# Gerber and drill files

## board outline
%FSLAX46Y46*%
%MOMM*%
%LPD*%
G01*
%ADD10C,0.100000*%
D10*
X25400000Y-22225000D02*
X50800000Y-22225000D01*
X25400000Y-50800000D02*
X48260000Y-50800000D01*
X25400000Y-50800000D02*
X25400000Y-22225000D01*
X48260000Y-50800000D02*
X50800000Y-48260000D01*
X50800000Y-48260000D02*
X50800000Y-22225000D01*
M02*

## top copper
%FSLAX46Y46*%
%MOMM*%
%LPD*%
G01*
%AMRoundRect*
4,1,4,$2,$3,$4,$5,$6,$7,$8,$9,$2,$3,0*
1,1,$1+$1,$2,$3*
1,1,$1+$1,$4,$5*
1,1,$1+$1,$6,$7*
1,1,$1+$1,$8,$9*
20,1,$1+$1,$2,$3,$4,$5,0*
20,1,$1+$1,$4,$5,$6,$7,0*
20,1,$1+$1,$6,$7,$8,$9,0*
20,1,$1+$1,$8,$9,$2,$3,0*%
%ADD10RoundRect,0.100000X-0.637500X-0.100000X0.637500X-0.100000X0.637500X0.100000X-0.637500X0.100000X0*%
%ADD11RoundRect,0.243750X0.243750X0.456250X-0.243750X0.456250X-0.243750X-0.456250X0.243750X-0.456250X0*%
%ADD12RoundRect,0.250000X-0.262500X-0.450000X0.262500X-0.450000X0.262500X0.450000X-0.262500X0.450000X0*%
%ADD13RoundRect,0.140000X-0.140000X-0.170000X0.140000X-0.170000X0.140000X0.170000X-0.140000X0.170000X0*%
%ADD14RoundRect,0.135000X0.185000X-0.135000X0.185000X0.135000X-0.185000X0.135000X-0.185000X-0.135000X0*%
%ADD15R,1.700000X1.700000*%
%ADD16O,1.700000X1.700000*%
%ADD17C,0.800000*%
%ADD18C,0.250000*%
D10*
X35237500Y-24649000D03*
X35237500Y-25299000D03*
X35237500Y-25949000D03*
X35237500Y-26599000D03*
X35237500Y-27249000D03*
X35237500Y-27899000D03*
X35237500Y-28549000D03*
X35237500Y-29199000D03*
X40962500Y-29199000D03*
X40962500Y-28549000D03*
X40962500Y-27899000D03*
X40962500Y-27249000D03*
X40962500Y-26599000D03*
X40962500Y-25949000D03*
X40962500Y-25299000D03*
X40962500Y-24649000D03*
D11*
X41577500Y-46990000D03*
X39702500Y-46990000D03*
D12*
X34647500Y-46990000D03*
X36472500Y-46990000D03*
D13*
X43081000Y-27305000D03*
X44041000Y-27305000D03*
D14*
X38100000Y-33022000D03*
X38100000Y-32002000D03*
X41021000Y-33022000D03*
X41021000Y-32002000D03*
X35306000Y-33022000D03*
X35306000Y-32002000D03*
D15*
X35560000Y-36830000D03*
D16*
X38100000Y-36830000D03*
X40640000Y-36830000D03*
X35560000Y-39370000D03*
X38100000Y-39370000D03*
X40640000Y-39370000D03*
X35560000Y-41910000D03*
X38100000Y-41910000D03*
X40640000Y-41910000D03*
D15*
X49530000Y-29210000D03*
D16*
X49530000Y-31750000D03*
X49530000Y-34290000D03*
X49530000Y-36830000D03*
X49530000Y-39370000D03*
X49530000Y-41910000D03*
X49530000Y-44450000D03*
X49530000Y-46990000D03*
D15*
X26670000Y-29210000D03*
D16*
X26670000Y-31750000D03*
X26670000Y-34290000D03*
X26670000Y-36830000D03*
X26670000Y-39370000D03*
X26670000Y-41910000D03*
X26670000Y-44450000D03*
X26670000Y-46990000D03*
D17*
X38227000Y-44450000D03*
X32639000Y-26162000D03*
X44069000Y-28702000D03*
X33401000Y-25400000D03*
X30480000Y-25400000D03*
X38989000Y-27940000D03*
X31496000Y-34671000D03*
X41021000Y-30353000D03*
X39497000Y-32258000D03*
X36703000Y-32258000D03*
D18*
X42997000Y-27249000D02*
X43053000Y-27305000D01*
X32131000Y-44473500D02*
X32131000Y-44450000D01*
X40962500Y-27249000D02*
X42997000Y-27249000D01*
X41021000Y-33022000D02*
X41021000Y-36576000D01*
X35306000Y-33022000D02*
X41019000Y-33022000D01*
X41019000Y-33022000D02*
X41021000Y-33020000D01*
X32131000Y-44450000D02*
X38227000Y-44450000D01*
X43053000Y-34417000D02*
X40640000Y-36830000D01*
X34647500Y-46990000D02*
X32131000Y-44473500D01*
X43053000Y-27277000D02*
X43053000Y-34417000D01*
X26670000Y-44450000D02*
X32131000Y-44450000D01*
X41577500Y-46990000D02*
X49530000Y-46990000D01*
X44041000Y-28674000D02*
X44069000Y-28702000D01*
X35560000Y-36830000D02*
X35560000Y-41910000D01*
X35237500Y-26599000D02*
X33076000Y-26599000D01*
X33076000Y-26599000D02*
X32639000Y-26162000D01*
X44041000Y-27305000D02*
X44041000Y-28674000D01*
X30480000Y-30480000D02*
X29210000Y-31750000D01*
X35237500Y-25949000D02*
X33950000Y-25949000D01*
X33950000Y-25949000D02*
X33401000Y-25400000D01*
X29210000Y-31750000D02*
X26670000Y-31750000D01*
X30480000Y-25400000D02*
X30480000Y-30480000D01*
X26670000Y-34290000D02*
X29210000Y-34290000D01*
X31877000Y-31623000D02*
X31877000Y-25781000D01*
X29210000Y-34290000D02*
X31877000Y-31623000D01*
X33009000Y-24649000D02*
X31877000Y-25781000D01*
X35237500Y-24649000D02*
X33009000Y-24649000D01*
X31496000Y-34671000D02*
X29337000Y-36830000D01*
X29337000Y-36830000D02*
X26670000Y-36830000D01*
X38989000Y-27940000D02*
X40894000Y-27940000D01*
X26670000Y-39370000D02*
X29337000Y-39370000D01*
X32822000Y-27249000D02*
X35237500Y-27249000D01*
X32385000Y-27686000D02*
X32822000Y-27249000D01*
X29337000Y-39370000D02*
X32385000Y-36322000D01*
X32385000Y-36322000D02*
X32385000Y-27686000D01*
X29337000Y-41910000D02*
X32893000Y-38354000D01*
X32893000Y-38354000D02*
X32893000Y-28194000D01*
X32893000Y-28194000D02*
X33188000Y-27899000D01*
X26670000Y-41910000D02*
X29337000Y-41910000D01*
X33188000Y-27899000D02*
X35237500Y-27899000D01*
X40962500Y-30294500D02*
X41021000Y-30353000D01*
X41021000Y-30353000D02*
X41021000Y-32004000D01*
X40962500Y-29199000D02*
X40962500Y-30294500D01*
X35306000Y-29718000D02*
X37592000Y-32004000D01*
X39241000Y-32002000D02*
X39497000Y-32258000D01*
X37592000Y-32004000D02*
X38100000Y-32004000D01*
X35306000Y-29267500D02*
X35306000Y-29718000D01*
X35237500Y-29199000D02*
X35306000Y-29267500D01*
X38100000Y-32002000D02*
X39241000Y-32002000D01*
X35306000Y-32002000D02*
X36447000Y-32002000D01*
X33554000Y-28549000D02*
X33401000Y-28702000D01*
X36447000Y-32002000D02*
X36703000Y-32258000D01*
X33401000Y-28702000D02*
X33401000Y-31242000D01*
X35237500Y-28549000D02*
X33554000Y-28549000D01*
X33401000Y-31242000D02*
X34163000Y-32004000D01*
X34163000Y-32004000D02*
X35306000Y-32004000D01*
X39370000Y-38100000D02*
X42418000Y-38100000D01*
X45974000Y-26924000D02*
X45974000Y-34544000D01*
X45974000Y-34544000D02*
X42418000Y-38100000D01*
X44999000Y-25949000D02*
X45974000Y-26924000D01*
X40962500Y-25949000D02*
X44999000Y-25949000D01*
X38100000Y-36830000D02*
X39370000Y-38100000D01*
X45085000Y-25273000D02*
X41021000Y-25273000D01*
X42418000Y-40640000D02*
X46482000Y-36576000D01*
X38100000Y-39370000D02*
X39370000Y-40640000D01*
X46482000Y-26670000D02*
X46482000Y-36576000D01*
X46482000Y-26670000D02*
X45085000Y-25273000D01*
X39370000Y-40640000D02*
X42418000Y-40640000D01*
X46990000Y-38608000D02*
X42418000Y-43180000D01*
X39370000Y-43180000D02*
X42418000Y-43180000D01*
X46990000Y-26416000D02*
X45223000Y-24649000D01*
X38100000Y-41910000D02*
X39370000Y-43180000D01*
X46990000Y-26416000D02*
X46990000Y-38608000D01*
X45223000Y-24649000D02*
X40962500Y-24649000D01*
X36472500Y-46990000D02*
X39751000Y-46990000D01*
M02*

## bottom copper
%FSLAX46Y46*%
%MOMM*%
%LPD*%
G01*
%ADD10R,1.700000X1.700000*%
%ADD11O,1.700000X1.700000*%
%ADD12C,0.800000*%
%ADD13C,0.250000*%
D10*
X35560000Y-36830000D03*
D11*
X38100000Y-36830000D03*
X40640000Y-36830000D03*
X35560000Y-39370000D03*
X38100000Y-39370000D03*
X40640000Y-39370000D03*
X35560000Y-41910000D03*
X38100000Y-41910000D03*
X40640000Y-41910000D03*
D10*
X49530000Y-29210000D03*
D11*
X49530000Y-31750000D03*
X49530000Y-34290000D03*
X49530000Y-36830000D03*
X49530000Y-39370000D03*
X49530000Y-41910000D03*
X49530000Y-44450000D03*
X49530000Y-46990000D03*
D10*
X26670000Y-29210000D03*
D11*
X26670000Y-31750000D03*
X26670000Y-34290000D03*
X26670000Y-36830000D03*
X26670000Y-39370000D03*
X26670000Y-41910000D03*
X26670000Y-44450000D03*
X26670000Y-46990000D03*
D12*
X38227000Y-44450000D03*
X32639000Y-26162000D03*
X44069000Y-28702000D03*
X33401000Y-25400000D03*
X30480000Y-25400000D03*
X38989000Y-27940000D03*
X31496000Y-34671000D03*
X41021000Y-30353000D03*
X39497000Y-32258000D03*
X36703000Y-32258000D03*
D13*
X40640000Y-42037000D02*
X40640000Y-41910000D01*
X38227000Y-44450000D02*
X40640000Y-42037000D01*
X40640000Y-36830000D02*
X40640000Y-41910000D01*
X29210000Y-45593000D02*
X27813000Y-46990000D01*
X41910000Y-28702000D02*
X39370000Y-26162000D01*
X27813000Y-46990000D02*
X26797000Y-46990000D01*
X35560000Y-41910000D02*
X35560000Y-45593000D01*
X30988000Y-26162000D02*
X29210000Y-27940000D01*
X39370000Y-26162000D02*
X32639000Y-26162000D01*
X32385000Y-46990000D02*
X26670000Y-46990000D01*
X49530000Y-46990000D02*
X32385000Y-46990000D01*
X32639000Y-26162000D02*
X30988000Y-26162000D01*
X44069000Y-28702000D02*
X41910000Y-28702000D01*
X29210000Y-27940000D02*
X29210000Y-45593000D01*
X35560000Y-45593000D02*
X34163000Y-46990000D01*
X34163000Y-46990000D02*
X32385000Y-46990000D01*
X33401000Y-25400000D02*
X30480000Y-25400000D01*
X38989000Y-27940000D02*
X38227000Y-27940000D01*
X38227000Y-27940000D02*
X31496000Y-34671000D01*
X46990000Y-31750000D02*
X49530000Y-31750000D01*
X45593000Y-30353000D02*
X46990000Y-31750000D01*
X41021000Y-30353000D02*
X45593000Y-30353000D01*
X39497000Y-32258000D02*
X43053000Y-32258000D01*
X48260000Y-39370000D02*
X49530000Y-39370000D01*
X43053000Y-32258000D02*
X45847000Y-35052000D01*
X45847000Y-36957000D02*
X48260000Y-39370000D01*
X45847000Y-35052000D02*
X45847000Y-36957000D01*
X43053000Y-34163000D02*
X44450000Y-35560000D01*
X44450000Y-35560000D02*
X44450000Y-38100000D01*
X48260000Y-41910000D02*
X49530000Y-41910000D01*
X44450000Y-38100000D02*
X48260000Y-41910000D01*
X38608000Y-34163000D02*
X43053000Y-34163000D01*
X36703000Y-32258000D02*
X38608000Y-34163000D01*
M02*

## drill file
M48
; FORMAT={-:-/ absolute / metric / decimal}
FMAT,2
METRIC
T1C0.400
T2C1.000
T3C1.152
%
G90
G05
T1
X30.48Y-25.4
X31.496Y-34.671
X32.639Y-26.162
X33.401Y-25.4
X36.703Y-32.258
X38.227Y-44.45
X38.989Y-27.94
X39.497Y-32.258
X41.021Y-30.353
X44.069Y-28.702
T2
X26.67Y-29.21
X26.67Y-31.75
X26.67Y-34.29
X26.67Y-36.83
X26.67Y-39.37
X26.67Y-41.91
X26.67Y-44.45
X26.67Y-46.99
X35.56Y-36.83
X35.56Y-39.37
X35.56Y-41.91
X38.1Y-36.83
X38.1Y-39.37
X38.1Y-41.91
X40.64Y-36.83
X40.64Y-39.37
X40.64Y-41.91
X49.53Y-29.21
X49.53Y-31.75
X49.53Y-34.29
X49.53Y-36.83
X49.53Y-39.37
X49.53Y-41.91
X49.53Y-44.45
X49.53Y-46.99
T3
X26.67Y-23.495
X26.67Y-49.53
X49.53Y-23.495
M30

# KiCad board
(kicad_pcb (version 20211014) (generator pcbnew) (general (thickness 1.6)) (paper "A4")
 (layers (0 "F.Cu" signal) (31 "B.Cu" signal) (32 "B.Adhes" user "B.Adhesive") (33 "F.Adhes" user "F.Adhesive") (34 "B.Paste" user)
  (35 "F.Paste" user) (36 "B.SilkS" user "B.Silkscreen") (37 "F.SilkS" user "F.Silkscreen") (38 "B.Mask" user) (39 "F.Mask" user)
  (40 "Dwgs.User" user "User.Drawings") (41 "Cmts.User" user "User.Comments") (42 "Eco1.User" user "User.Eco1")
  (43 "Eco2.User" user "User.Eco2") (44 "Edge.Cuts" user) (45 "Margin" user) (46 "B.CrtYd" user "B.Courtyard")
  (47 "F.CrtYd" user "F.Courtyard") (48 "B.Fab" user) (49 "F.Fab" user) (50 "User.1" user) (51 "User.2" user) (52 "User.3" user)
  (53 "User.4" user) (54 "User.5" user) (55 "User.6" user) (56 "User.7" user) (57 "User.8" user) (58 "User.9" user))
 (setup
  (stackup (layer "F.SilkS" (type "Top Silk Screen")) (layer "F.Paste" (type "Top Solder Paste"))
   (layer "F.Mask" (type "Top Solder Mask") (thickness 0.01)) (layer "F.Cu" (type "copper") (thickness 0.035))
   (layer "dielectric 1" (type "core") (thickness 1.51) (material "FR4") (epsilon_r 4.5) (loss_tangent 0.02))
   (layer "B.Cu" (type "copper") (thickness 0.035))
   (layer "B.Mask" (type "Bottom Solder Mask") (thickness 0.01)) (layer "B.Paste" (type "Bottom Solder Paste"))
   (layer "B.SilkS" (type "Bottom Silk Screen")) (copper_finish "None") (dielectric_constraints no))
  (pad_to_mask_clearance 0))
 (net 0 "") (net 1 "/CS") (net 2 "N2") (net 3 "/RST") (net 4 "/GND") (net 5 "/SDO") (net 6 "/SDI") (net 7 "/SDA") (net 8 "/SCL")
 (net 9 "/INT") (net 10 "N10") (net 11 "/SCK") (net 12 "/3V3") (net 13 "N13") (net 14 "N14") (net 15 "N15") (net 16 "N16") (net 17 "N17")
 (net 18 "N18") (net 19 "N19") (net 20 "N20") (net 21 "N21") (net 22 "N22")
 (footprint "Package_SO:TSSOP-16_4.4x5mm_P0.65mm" (layer "F.Cu") (at 38.1 26.924)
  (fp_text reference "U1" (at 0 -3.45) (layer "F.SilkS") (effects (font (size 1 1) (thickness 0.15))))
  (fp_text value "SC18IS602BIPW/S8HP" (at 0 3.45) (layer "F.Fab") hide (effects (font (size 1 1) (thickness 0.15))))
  (pad "1" smd roundrect (at -2.8625 -2.275) (size 1.475 0.4) (layers "F.Cu" "F.Paste" "F.Mask") (roundrect_rratio 0.25) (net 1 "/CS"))
  (pad "2" smd roundrect (at -2.8625 -1.625) (size 1.475 0.4) (layers "F.Cu" "F.Paste" "F.Mask") (roundrect_rratio 0.25) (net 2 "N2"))
  (pad "3" smd roundrect (at -2.8625 -0.975) (size 1.475 0.4) (layers "F.Cu" "F.Paste" "F.Mask") (roundrect_rratio 0.25) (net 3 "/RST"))
  (pad "4" smd roundrect (at -2.8625 -0.325) (size 1.475 0.4) (layers "F.Cu" "F.Paste" "F.Mask") (roundrect_rratio 0.25) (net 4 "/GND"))
  (pad "5" smd roundrect (at -2.8625 0.325) (size 1.475 0.4) (layers "F.Cu" "F.Paste" "F.Mask") (roundrect_rratio 0.25) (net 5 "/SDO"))
  (pad "6" smd roundrect (at -2.8625 0.975) (size 1.475 0.4) (layers "F.Cu" "F.Paste" "F.Mask") (roundrect_rratio 0.25) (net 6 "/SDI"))
  (pad "7" smd roundrect (at -2.8625 1.625) (size 1.475 0.4) (layers "F.Cu" "F.Paste" "F.Mask") (roundrect_rratio 0.25) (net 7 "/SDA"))
  (pad "8" smd roundrect (at -2.8625 2.275) (size 1.475 0.4) (layers "F.Cu" "F.Paste" "F.Mask") (roundrect_rratio 0.25) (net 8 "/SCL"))
  (pad "9" smd roundrect (at 2.8625 2.275) (size 1.475 0.4) (layers "F.Cu" "F.Paste" "F.Mask") (roundrect_rratio 0.25) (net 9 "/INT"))
  (pad "10" smd roundrect (at 2.8625 1.625) (size 1.475 0.4) (layers "F.Cu" "F.Paste" "F.Mask") (roundrect_rratio 0.25) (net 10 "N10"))
  (pad "11" smd roundrect (at 2.8625 0.975) (size 1.475 0.4) (layers "F.Cu" "F.Paste" "F.Mask") (roundrect_rratio 0.25) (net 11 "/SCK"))
  (pad "12" smd roundrect (at 2.8625 0.325) (size 1.475 0.4) (layers "F.Cu" "F.Paste" "F.Mask") (roundrect_rratio 0.25) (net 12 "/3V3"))
  (pad "13" smd roundrect (at 2.8625 -0.325) (size 1.475 0.4) (layers "F.Cu" "F.Paste" "F.Mask") (roundrect_rratio 0.25) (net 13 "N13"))
  (pad "14" smd roundrect (at 2.8625 -0.975) (size 1.475 0.4) (layers "F.Cu" "F.Paste" "F.Mask") (roundrect_rratio 0.25) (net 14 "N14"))
  (pad "15" smd roundrect (at 2.8625 -1.625) (size 1.475 0.4) (layers "F.Cu" "F.Paste" "F.Mask") (roundrect_rratio 0.25) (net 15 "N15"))
  (pad "16" smd roundrect (at 2.8625 -2.275) (size 1.475 0.4) (layers "F.Cu" "F.Paste" "F.Mask") (roundrect_rratio 0.25) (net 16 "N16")))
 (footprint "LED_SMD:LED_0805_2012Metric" (layer "F.Cu") (at 40.64 46.99 180)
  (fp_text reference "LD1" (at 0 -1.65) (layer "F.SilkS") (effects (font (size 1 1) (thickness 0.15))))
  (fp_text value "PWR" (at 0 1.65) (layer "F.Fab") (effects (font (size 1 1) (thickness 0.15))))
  (pad "1" smd roundrect (at -0.9375 0 180) (size 0.975 1.4) (layers "F.Cu" "F.Paste" "F.Mask") (roundrect_rratio 0.25) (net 4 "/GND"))
  (pad "2" smd roundrect (at 0.9375 0 180) (size 0.975 1.4) (layers "F.Cu" "F.Paste" "F.Mask") (roundrect_rratio 0.25) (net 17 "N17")))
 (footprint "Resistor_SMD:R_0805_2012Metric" (layer "F.Cu") (at 35.56 46.99)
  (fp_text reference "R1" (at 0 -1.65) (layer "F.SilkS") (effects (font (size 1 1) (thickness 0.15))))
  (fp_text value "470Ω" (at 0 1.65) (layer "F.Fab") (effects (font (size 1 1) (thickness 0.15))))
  (pad "1" smd roundrect (at -0.9125 0) (size 1.025 1.4) (layers "F.Cu" "F.Paste" "F.Mask") (roundrect_rratio 0.243902) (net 12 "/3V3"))
  (pad "2" smd roundrect (at 0.9125 0) (size 1.025 1.4) (layers "F.Cu" "F.Paste" "F.Mask") (roundrect_rratio 0.243902) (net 17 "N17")))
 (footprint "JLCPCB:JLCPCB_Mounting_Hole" (layer "F.Cu") (at 49.53 23.495)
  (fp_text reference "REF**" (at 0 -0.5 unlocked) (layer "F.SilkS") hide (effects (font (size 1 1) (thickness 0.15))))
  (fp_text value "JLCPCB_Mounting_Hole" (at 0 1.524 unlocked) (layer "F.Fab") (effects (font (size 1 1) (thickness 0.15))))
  (pad "" np_thru_hole circle (at 0 0) (size 1.152 1.152) (drill 1.152) (layers F&B.Cu *.Mask) (solder_mask_margin 0.148)))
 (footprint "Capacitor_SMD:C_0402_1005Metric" (layer "F.Cu") (at 43.561 27.305)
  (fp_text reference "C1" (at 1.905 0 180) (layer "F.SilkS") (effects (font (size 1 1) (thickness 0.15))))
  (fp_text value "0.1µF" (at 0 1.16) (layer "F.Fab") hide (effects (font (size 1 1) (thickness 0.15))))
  (pad "1" smd roundrect (at -0.48 0) (size 0.56 0.62) (layers "F.Cu" "F.Paste" "F.Mask") (roundrect_rratio 0.25) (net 12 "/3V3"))
  (pad "2" smd roundrect (at 0.48 0) (size 0.56 0.62) (layers "F.Cu" "F.Paste" "F.Mask") (roundrect_rratio 0.25) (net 4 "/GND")))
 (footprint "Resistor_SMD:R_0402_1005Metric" (layer "F.Cu") (at 38.1 32.512 90)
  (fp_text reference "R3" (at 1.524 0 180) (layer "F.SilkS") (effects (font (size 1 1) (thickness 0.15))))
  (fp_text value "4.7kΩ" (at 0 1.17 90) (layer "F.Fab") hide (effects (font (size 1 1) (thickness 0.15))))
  (pad "1" smd roundrect (at -0.51 0 90) (size 0.54 0.64) (layers "F.Cu" "F.Paste" "F.Mask") (roundrect_rratio 0.25) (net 12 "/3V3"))
  (pad "2" smd roundrect (at 0.51 0 90) (size 0.54 0.64) (layers "F.Cu" "F.Paste" "F.Mask") (roundrect_rratio 0.25) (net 8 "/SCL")))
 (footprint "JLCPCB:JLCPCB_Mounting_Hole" (layer "F.Cu") (at 26.67 23.495)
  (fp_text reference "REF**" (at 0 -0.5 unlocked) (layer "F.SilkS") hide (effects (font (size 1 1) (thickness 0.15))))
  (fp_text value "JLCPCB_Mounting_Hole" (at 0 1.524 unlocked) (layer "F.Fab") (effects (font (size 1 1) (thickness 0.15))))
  (pad "" np_thru_hole circle (at 0 0) (size 1.152 1.152) (drill 1.152) (layers F&B.Cu *.Mask) (solder_mask_margin 0.148)))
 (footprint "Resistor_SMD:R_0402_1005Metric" (layer "F.Cu") (at 41.021 32.512 90)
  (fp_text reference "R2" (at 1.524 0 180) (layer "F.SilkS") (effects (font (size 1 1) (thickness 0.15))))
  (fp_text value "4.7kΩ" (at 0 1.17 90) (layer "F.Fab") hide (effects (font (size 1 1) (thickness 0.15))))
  (pad "1" smd roundrect (at -0.51 0 90) (size 0.54 0.64) (layers "F.Cu" "F.Paste" "F.Mask") (roundrect_rratio 0.25) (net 12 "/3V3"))
  (pad "2" smd roundrect (at 0.51 0 90) (size 0.54 0.64) (layers "F.Cu" "F.Paste" "F.Mask") (roundrect_rratio 0.25) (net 9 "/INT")))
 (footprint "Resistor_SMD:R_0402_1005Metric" (layer "F.Cu") (at 35.306 32.512 90)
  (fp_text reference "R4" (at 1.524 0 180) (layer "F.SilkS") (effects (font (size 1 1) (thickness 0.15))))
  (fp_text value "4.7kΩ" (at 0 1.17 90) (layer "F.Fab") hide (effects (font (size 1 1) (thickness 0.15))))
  (pad "1" smd roundrect (at -0.51 0 90) (size 0.54 0.64) (layers "F.Cu" "F.Paste" "F.Mask") (roundrect_rratio 0.25) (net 12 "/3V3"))
  (pad "2" smd roundrect (at 0.51 0 90) (size 0.54 0.64) (layers "F.Cu" "F.Paste" "F.Mask") (roundrect_rratio 0.25) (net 7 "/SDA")))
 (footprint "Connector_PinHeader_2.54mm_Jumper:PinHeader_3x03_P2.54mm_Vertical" (layer "F.Cu") (at 35.56 36.83)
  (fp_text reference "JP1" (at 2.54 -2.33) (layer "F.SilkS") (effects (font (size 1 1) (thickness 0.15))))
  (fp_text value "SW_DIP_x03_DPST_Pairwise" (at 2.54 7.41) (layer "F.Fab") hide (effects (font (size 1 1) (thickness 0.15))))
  (pad "1" thru_hole rect (at 0 0) (size 1.7 1.7) (drill 1) (layers *.Cu *.Mask) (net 4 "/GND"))
  (pad "2" thru_hole oval (at 2.54 0) (size 1.7 1.7) (drill 1) (layers *.Cu *.Mask) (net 14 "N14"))
  (pad "3" thru_hole oval (at 5.08 0) (size 1.7 1.7) (drill 1) (layers *.Cu *.Mask) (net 12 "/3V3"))
  (pad "4" thru_hole oval (at 0 2.54) (size 1.7 1.7) (drill 1) (layers *.Cu *.Mask) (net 4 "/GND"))
  (pad "5" thru_hole oval (at 2.54 2.54) (size 1.7 1.7) (drill 1) (layers *.Cu *.Mask) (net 15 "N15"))
  (pad "6" thru_hole oval (at 5.08 2.54) (size 1.7 1.7) (drill 1) (layers *.Cu *.Mask) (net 12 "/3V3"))
  (pad "7" thru_hole oval (at 0 5.08) (size 1.7 1.7) (drill 1) (layers *.Cu *.Mask) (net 4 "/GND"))
  (pad "8" thru_hole oval (at 2.54 5.08) (size 1.7 1.7) (drill 1) (layers *.Cu *.Mask) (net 16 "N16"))
  (pad "9" thru_hole oval (at 5.08 5.08) (size 1.7 1.7) (drill 1) (layers *.Cu *.Mask) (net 12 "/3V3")))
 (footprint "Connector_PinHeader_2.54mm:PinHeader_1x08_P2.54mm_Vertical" (layer "F.Cu") (at 49.53 29.21)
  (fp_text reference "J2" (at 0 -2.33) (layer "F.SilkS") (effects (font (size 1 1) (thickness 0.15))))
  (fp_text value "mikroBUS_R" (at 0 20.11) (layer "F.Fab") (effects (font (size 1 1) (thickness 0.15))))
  (pad "1" thru_hole rect (at 0 0) (size 1.7 1.7) (drill 1) (layers *.Cu *.Mask) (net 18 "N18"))
  (pad "2" thru_hole oval (at 0 2.54) (size 1.7 1.7) (drill 1) (layers *.Cu *.Mask) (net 9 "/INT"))
  (pad "3" thru_hole oval (at 0 5.08) (size 1.7 1.7) (drill 1) (layers *.Cu *.Mask) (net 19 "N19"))
  (pad "4" thru_hole oval (at 0 7.62) (size 1.7 1.7) (drill 1) (layers *.Cu *.Mask) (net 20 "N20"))
  (pad "5" thru_hole oval (at 0 10.16) (size 1.7 1.7) (drill 1) (layers *.Cu *.Mask) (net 8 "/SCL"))
  (pad "6" thru_hole oval (at 0 12.7) (size 1.7 1.7) (drill 1) (layers *.Cu *.Mask) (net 7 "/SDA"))
  (pad "7" thru_hole oval (at 0 15.24) (size 1.7 1.7) (drill 1) (layers *.Cu *.Mask) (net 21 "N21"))
  (pad "8" thru_hole oval (at 0 17.78) (size 1.7 1.7) (drill 1) (layers *.Cu *.Mask) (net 4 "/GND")))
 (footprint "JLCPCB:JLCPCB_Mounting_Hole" (layer "F.Cu") (at 26.67 49.53)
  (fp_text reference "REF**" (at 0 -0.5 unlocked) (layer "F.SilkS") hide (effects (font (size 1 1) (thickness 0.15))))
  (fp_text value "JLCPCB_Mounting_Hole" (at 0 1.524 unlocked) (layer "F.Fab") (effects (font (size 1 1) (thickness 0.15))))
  (pad "" np_thru_hole circle (at 0 0) (size 1.152 1.152) (drill 1.152) (layers F&B.Cu *.Mask) (solder_mask_margin 0.148)))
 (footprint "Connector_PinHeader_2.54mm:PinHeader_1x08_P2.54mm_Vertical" (layer "F.Cu") (at 26.67 29.21)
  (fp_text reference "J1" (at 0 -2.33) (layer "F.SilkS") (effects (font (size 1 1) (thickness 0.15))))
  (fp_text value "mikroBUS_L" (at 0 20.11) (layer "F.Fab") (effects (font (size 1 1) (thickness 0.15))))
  (pad "1" thru_hole rect (at 0 0) (size 1.7 1.7) (drill 1) (layers *.Cu *.Mask) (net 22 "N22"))
  (pad "2" thru_hole oval (at 0 2.54) (size 1.7 1.7) (drill 1) (layers *.Cu *.Mask) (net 3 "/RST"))
  (pad "3" thru_hole oval (at 0 5.08) (size 1.7 1.7) (drill 1) (layers *.Cu *.Mask) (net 1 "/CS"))
  (pad "4" thru_hole oval (at 0 7.62) (size 1.7 1.7) (drill 1) (layers *.Cu *.Mask) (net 11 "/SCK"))
  (pad "5" thru_hole oval (at 0 10.16) (size 1.7 1.7) (drill 1) (layers *.Cu *.Mask) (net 5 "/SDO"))
  (pad "6" thru_hole oval (at 0 12.7) (size 1.7 1.7) (drill 1) (layers *.Cu *.Mask) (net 6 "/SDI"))
  (pad "7" thru_hole oval (at 0 15.24) (size 1.7 1.7) (drill 1) (layers *.Cu *.Mask) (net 12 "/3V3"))
  (pad "8" thru_hole oval (at 0 17.78) (size 1.7 1.7) (drill 1) (layers *.Cu *.Mask) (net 4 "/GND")))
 (gr_line (start 25.4 22.225) (end 50.8 22.225) (layer "Edge.Cuts") (width 0.1))
 (gr_line (start 25.4 50.8) (end 48.26 50.8) (layer "Edge.Cuts") (width 0.1))
 (gr_line (start 25.4 50.8) (end 25.4 22.225) (layer "Edge.Cuts") (width 0.1))
 (gr_line (start 48.26 50.8) (end 50.8 48.26) (layer "Edge.Cuts") (width 0.1))
 (gr_line (start 50.8 48.26) (end 50.8 22.225) (layer "Edge.Cuts") (width 0.1))
 (segment (start 42.997 27.249) (end 43.053 27.305) (width 0.25) (layer "F.Cu") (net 12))
 (segment (start 32.131 44.4735) (end 32.131 44.45) (width 0.25) (layer "F.Cu") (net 12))
 (segment (start 40.9625 27.249) (end 42.997 27.249) (width 0.25) (layer "F.Cu") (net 12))
 (segment (start 41.021 33.022) (end 41.021 36.576) (width 0.25) (layer "F.Cu") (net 12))
 (segment (start 35.306 33.022) (end 41.019 33.022) (width 0.25) (layer "F.Cu") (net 12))
 (segment (start 41.019 33.022) (end 41.021 33.02) (width 0.25) (layer "F.Cu") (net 12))
 (segment (start 32.131 44.45) (end 38.227 44.45) (width 0.25) (layer "F.Cu") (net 12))
 (segment (start 43.053 34.417) (end 40.64 36.83) (width 0.25) (layer "F.Cu") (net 12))
 (segment (start 34.6475 46.99) (end 32.131 44.4735) (width 0.25) (layer "F.Cu") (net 12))
 (segment (start 43.053 27.277) (end 43.053 34.417) (width 0.25) (layer "F.Cu") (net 12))
 (segment (start 26.67 44.45) (end 32.131 44.45) (width 0.25) (layer "F.Cu") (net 12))
 (via (at 38.227 44.45) (size 0.8) (drill 0.4) (layers "F.Cu" "B.Cu") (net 12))
 (segment (start 40.64 42.037) (end 40.64 41.91) (width 0.25) (layer "B.Cu") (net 12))
 (segment (start 38.227 44.45) (end 40.64 42.037) (width 0.25) (layer "B.Cu") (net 12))
 (segment (start 40.64 36.83) (end 40.64 41.91) (width 0.25) (layer "B.Cu") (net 12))
 (segment (start 41.5775 46.99) (end 49.53 46.99) (width 0.25) (layer "F.Cu") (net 4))
 (segment (start 44.041 28.674) (end 44.069 28.702) (width 0.25) (layer "F.Cu") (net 4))
 (segment (start 35.56 36.83) (end 35.56 41.91) (width 0.25) (layer "F.Cu") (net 4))
 (segment (start 35.2375 26.599) (end 33.076 26.599) (width 0.25) (layer "F.Cu") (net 4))
 (segment (start 33.076 26.599) (end 32.639 26.162) (width 0.25) (layer "F.Cu") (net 4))
 (segment (start 44.041 27.305) (end 44.041 28.674) (width 0.25) (layer "F.Cu") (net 4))
 (via (at 32.639 26.162) (size 0.8) (drill 0.4) (layers "F.Cu" "B.Cu") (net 4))
 (via (at 44.069 28.702) (size 0.8) (drill 0.4) (layers "F.Cu" "B.Cu") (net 4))
 (segment (start 29.21 45.593) (end 27.813 46.99) (width 0.25) (layer "B.Cu") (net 4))
 (segment (start 41.91 28.702) (end 39.37 26.162) (width 0.25) (layer "B.Cu") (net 4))
 (segment (start 27.813 46.99) (end 26.797 46.99) (width 0.25) (layer "B.Cu") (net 4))
 (segment (start 35.56 41.91) (end 35.56 45.593) (width 0.25) (layer "B.Cu") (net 4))
 (segment (start 30.988 26.162) (end 29.21 27.94) (width 0.25) (layer "B.Cu") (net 4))
 (segment (start 39.37 26.162) (end 32.639 26.162) (width 0.25) (layer "B.Cu") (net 4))
 (segment (start 32.385 46.99) (end 26.67 46.99) (width 0.25) (layer "B.Cu") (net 4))
 (segment (start 49.53 46.99) (end 32.385 46.99) (width 0.25) (layer "B.Cu") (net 4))
 (segment (start 32.639 26.162) (end 30.988 26.162) (width 0.25) (layer "B.Cu") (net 4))
 (segment (start 44.069 28.702) (end 41.91 28.702) (width 0.25) (layer "B.Cu") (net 4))
 (segment (start 29.21 27.94) (end 29.21 45.593) (width 0.25) (layer "B.Cu") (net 4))
 (segment (start 35.56 45.593) (end 34.163 46.99) (width 0.25) (layer "B.Cu") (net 4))
 (segment (start 34.163 46.99) (end 32.385 46.99) (width 0.25) (layer "B.Cu") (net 4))
 (segment (start 30.48 30.48) (end 29.21 31.75) (width 0.25) (layer "F.Cu") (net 3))
 (segment (start 35.2375 25.949) (end 33.95 25.949) (width 0.25) (layer "F.Cu") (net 3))
 (segment (start 33.95 25.949) (end 33.401 25.4) (width 0.25) (layer "F.Cu") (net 3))
 (segment (start 29.21 31.75) (end 26.67 31.75) (width 0.25) (layer "F.Cu") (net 3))
 (segment (start 30.48 25.4) (end 30.48 30.48) (width 0.25) (layer "F.Cu") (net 3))
 (via (at 33.401 25.4) (size 0.8) (drill 0.4) (layers "F.Cu" "B.Cu") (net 3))
 (via (at 30.48 25.4) (size 0.8) (drill 0.4) (layers "F.Cu" "B.Cu") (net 3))
 (segment (start 33.401 25.4) (end 30.48 25.4) (width 0.25) (layer "B.Cu") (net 3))
 (segment (start 26.67 34.29) (end 29.21 34.29) (width 0.25) (layer "F.Cu") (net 1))
 (segment (start 31.877 31.623) (end 31.877 25.781) (width 0.25) (layer "F.Cu") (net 1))
 (segment (start 29.21 34.29) (end 31.877 31.623) (width 0.25) (layer "F.Cu") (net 1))
 (segment (start 33.009 24.649) (end 31.877 25.781) (width 0.25) (layer "F.Cu") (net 1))
 (segment (start 35.2375 24.649) (end 33.009 24.649) (width 0.25) (layer "F.Cu") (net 1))
 (segment (start 31.496 34.671) (end 29.337 36.83) (width 0.25) (layer "F.Cu") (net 11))
 (segment (start 29.337 36.83) (end 26.67 36.83) (width 0.25) (layer "F.Cu") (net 11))
 (segment (start 38.989 27.94) (end 40.894 27.94) (width 0.25) (layer "F.Cu") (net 11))
 (via (at 38.989 27.94) (size 0.8) (drill 0.4) (layers "F.Cu" "B.Cu") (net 11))
 (via (at 31.496 34.671) (size 0.8) (drill 0.4) (layers "F.Cu" "B.Cu") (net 11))
 (segment (start 38.989 27.94) (end 38.227 27.94) (width 0.25) (layer "B.Cu") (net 11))
 (segment (start 38.227 27.94) (end 31.496 34.671) (width 0.25) (layer "B.Cu") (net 11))
 (segment (start 26.67 39.37) (end 29.337 39.37) (width 0.25) (layer "F.Cu") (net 5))
 (segment (start 32.822 27.249) (end 35.2375 27.249) (width 0.25) (layer "F.Cu") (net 5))
 (segment (start 32.385 27.686) (end 32.822 27.249) (width 0.25) (layer "F.Cu") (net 5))
 (segment (start 29.337 39.37) (end 32.385 36.322) (width 0.25) (layer "F.Cu") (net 5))
 (segment (start 32.385 36.322) (end 32.385 27.686) (width 0.25) (layer "F.Cu") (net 5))
 (segment (start 29.337 41.91) (end 32.893 38.354) (width 0.25) (layer "F.Cu") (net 6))
 (segment (start 32.893 38.354) (end 32.893 28.194) (width 0.25) (layer "F.Cu") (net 6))
 (segment (start 32.893 28.194) (end 33.188 27.899) (width 0.25) (layer "F.Cu") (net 6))
 (segment (start 26.67 41.91) (end 29.337 41.91) (width 0.25) (layer "F.Cu") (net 6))
 (segment (start 33.188 27.899) (end 35.2375 27.899) (width 0.25) (layer "F.Cu") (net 6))
 (segment (start 40.9625 30.2945) (end 41.021 30.353) (width 0.25) (layer "F.Cu") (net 9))
 (segment (start 41.021 30.353) (end 41.021 32.004) (width 0.25) (layer "F.Cu") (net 9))
 (segment (start 40.9625 29.199) (end 40.9625 30.2945) (width 0.25) (layer "F.Cu") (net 9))
 (via (at 41.021 30.353) (size 0.8) (drill 0.4) (layers "F.Cu" "B.Cu") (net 9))
 (segment (start 46.99 31.75) (end 49.53 31.75) (width 0.25) (layer "B.Cu") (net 9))
 (segment (start 45.593 30.353) (end 46.99 31.75) (width 0.25) (layer "B.Cu") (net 9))
 (segment (start 41.021 30.353) (end 45.593 30.353) (width 0.25) (layer "B.Cu") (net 9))
 (segment (start 35.306 29.718) (end 37.592 32.004) (width 0.25) (layer "F.Cu") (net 8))
 (segment (start 39.241 32.002) (end 39.497 32.258) (width 0.25) (layer "F.Cu") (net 8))
 (segment (start 37.592 32.004) (end 38.1 32.004) (width 0.25) (layer "F.Cu") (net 8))
 (segment (start 35.306 29.2675) (end 35.306 29.718) (width 0.25) (layer "F.Cu") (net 8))
 (segment (start 35.2375 29.199) (end 35.306 29.2675) (width 0.25) (layer "F.Cu") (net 8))
 (segment (start 38.1 32.002) (end 39.241 32.002) (width 0.25) (layer "F.Cu") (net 8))
 (via (at 39.497 32.258) (size 0.8) (drill 0.4) (layers "F.Cu" "B.Cu") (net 8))
 (segment (start 39.497 32.258) (end 43.053 32.258) (width 0.25) (layer "B.Cu") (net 8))
 (segment (start 48.26 39.37) (end 49.53 39.37) (width 0.25) (layer "B.Cu") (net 8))
 (segment (start 43.053 32.258) (end 45.847 35.052) (width 0.25) (layer "B.Cu") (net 8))
 (segment (start 45.847 36.957) (end 48.26 39.37) (width 0.25) (layer "B.Cu") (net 8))
 (segment (start 45.847 35.052) (end 45.847 36.957) (width 0.25) (layer "B.Cu") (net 8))
 (segment (start 35.306 32.002) (end 36.447 32.002) (width 0.25) (layer "F.Cu") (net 7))
 (segment (start 33.554 28.549) (end 33.401 28.702) (width 0.25) (layer "F.Cu") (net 7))
 (segment (start 36.447 32.002) (end 36.703 32.258) (width 0.25) (layer "F.Cu") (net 7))
 (segment (start 33.401 28.702) (end 33.401 31.242) (width 0.25) (layer "F.Cu") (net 7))
 (segment (start 35.2375 28.549) (end 33.554 28.549) (width 0.25) (layer "F.Cu") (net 7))
 (segment (start 33.401 31.242) (end 34.163 32.004) (width 0.25) (layer "F.Cu") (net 7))
 (segment (start 34.163 32.004) (end 35.306 32.004) (width 0.25) (layer "F.Cu") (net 7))
 (via (at 36.703 32.258) (size 0.8) (drill 0.4) (layers "F.Cu" "B.Cu") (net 7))
 (segment (start 43.053 34.163) (end 44.45 35.56) (width 0.25) (layer "B.Cu") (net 7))
 (segment (start 44.45 35.56) (end 44.45 38.1) (width 0.25) (layer "B.Cu") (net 7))
 (segment (start 48.26 41.91) (end 49.53 41.91) (width 0.25) (layer "B.Cu") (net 7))
 (segment (start 44.45 38.1) (end 48.26 41.91) (width 0.25) (layer "B.Cu") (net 7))
 (segment (start 38.608 34.163) (end 43.053 34.163) (width 0.25) (layer "B.Cu") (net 7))
 (segment (start 36.703 32.258) (end 38.608 34.163) (width 0.25) (layer "B.Cu") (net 7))
 (segment (start 39.37 38.1) (end 42.418 38.1) (width 0.25) (layer "F.Cu") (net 14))
 (segment (start 45.974 26.924) (end 45.974 34.544) (width 0.25) (layer "F.Cu") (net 14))
 (segment (start 45.974 34.544) (end 42.418 38.1) (width 0.25) (layer "F.Cu") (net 14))
 (segment (start 44.999 25.949) (end 45.974 26.924) (width 0.25) (layer "F.Cu") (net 14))
 (segment (start 40.9625 25.949) (end 44.999 25.949) (width 0.25) (layer "F.Cu") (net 14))
 (segment (start 38.1 36.83) (end 39.37 38.1) (width 0.25) (layer "F.Cu") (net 14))
 (segment (start 45.085 25.273) (end 41.021 25.273) (width 0.25) (layer "F.Cu") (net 15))
 (segment (start 42.418 40.64) (end 46.482 36.576) (width 0.25) (layer "F.Cu") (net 15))
 (segment (start 38.1 39.37) (end 39.37 40.64) (width 0.25) (layer "F.Cu") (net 15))
 (segment (start 46.482 26.67) (end 46.482 36.576) (width 0.25) (layer "F.Cu") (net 15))
 (segment (start 46.482 26.67) (end 45.085 25.273) (width 0.25) (layer "F.Cu") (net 15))
 (segment (start 39.37 40.64) (end 42.418 40.64) (width 0.25) (layer "F.Cu") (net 15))
 (segment (start 46.99 38.608) (end 42.418 43.18) (width 0.25) (layer "F.Cu") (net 16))
 (segment (start 39.37 43.18) (end 42.418 43.18) (width 0.25) (layer "F.Cu") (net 16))
 (segment (start 46.99 26.416) (end 45.223 24.649) (width 0.25) (layer "F.Cu") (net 16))
 (segment (start 38.1 41.91) (end 39.37 43.18) (width 0.25) (layer "F.Cu") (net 16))
 (segment (start 46.99 26.416) (end 46.99 38.608) (width 0.25) (layer "F.Cu") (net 16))
 (segment (start 45.223 24.649) (end 40.9625 24.649) (width 0.25) (layer "F.Cu") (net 16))
 (segment (start 36.4725 46.99) (end 39.751 46.99) (width 0.25) (layer "F.Cu") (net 17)))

